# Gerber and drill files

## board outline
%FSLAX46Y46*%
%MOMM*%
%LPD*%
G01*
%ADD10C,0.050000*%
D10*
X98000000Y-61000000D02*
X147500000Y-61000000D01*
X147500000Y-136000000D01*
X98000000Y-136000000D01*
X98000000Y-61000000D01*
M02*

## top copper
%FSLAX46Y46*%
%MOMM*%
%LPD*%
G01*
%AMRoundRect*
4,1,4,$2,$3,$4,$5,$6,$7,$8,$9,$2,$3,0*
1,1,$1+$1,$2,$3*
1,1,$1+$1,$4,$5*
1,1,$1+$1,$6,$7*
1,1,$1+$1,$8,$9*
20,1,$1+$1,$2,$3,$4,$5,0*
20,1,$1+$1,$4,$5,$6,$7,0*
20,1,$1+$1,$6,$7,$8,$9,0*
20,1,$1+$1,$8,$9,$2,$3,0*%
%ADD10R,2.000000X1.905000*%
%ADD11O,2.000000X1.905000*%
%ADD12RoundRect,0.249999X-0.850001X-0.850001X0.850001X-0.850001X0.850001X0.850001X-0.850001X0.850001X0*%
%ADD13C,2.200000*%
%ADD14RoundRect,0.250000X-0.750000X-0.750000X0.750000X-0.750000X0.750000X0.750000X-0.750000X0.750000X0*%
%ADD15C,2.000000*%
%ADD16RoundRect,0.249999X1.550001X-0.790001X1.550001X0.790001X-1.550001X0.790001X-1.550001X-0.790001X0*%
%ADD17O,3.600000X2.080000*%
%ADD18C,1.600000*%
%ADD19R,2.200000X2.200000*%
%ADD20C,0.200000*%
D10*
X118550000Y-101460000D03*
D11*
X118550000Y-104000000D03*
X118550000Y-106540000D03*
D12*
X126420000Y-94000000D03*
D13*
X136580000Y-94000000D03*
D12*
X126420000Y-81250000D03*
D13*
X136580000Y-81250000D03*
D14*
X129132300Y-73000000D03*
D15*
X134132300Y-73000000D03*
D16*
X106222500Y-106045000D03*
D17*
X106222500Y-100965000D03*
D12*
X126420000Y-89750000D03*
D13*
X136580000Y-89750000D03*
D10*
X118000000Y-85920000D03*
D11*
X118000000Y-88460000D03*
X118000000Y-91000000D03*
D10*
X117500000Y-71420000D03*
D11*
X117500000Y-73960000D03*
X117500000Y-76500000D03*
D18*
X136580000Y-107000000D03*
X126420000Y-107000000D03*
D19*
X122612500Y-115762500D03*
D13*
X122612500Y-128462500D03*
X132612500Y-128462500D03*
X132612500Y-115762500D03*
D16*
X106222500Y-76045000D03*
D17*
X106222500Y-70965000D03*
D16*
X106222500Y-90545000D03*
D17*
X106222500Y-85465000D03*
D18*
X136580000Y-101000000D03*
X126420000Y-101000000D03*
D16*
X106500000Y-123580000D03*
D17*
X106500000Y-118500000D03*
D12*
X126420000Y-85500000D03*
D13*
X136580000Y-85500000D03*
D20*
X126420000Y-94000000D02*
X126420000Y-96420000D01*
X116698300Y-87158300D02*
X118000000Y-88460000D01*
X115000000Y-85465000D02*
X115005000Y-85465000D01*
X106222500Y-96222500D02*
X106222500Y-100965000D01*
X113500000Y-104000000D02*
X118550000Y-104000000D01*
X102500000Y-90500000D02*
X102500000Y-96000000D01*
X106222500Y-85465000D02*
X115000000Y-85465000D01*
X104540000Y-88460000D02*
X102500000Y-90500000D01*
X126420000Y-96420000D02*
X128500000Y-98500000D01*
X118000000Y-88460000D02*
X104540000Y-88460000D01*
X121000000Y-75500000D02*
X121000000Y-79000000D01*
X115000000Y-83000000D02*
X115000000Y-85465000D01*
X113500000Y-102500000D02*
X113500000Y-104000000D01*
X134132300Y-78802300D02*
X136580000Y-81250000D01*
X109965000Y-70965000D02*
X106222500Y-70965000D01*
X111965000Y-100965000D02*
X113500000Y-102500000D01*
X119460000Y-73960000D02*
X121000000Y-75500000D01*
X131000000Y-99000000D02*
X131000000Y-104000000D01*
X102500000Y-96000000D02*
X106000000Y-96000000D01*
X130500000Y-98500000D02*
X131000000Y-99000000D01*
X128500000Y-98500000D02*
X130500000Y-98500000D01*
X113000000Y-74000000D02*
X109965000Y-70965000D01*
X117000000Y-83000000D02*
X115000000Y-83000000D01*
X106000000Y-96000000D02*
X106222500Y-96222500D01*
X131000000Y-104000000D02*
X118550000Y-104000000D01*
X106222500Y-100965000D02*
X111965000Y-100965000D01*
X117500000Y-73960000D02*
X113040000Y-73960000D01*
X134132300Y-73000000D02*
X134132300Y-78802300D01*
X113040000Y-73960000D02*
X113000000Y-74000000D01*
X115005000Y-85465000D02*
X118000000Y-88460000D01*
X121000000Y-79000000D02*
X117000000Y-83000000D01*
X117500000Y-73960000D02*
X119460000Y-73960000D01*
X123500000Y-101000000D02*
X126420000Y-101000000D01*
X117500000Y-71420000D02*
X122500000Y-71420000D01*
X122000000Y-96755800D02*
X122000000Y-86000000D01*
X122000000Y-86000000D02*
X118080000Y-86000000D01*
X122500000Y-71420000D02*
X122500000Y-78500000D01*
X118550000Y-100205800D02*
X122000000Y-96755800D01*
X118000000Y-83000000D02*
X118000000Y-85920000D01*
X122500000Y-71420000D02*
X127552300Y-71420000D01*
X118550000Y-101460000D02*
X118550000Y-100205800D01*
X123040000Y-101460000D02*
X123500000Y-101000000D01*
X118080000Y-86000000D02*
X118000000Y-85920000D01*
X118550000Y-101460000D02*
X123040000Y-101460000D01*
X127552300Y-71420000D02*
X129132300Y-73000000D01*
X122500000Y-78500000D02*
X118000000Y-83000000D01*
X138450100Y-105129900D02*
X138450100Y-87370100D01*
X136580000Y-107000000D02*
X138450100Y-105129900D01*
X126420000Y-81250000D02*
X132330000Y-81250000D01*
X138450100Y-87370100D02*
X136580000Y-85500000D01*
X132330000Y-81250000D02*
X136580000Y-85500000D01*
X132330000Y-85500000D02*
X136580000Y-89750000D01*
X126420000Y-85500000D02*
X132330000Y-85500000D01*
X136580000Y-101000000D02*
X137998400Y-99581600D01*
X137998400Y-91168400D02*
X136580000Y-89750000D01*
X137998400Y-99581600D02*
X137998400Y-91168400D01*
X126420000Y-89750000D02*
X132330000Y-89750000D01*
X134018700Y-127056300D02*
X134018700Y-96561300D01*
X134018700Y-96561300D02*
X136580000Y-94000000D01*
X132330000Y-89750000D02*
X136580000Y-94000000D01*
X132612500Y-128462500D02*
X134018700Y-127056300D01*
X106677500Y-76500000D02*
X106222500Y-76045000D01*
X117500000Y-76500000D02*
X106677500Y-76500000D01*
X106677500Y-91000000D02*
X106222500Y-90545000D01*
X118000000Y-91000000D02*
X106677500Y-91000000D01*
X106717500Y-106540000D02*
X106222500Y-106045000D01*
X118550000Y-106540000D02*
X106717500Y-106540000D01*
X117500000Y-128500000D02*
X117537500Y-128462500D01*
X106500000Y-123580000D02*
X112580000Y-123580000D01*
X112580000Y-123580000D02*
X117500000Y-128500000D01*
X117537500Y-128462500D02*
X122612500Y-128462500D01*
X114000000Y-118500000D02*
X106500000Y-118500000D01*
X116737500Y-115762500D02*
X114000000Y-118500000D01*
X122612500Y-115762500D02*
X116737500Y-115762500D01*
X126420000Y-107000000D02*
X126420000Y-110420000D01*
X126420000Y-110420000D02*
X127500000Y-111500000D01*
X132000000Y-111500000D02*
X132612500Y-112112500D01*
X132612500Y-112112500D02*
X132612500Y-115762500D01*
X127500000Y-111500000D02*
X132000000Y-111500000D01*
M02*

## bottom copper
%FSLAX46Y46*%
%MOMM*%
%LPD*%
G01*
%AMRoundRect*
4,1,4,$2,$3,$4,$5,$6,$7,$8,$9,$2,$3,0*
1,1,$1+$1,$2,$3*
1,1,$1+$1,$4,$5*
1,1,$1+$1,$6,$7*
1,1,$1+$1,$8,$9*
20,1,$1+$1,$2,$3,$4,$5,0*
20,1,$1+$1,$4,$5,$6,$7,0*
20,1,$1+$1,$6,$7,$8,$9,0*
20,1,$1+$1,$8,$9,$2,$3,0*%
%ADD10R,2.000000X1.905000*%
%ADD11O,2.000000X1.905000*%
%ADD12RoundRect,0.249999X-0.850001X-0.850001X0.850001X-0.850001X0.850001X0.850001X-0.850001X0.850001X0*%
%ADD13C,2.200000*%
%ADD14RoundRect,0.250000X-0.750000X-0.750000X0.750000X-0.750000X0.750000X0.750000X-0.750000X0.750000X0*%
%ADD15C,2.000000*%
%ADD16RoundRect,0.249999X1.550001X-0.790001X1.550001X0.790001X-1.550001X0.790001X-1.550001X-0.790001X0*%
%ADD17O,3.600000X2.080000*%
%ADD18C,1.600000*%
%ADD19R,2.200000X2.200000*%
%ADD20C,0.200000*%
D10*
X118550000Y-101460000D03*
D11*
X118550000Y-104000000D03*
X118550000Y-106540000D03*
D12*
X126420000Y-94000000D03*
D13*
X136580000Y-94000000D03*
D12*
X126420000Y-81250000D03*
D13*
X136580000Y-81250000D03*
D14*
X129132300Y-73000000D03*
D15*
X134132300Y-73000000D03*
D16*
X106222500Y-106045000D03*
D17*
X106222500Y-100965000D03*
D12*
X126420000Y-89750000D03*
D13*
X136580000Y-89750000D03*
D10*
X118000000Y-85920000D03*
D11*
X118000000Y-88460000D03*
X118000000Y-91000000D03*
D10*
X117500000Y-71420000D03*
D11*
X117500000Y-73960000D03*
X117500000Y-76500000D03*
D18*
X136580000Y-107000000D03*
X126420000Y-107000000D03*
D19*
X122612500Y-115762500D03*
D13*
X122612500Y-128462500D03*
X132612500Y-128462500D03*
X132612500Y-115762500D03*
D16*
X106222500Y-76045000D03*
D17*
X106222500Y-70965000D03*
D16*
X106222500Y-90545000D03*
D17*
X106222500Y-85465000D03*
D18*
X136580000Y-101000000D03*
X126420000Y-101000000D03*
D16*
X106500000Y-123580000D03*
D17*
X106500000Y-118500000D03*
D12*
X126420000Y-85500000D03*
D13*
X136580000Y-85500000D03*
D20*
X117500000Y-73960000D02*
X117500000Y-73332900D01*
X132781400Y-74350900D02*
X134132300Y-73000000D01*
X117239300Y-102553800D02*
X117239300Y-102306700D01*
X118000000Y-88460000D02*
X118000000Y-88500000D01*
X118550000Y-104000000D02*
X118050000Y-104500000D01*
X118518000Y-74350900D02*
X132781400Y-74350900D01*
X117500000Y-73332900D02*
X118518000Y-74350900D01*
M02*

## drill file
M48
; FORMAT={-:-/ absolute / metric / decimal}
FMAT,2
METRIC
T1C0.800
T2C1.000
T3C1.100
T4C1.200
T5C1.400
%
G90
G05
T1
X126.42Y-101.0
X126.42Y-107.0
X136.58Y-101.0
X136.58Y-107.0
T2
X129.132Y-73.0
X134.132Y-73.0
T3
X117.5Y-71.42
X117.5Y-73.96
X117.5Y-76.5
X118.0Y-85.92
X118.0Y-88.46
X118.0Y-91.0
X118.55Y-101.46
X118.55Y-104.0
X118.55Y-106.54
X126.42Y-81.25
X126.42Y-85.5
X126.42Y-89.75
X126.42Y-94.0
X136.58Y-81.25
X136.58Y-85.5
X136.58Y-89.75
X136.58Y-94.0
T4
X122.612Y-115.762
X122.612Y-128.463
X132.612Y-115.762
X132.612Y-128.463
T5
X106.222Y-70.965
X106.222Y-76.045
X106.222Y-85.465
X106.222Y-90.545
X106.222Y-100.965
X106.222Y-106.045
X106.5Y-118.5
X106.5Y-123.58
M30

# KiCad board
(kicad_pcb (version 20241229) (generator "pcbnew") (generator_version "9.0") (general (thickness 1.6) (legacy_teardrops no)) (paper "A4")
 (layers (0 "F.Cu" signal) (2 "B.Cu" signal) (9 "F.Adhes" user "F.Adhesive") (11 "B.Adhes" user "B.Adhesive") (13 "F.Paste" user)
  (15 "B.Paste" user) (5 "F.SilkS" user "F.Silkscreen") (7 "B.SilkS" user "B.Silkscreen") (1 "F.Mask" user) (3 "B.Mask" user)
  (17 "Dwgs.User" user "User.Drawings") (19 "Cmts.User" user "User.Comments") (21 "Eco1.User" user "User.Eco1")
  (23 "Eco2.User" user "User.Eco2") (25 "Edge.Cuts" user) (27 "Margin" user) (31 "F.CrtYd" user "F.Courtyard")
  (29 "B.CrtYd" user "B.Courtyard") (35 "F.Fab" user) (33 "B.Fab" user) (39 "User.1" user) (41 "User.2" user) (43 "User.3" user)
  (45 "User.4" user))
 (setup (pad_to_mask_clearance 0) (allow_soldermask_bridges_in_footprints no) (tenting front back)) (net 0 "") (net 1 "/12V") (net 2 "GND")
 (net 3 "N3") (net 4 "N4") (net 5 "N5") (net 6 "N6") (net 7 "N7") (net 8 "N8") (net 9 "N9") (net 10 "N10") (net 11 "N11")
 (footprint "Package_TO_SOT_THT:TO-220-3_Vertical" (layer "F.Cu") (at 118.55 101.46 -90)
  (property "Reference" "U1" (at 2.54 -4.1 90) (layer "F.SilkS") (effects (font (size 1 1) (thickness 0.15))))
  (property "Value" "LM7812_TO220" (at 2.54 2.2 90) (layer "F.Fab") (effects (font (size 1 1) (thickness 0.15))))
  (pad "1" thru_hole rect (at 0 0 270) (size 1.905 2) (drill 1.1) (layers "*.Cu" "*.Mask") (remove_unused_layers no) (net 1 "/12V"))
  (pad "2" thru_hole oval (at 2.54 0 270) (size 1.905 2) (drill 1.1) (layers "*.Cu" "*.Mask") (remove_unused_layers no) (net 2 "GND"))
  (pad "3" thru_hole oval (at 5.08 0 270) (size 1.905 2) (drill 1.1) (layers "*.Cu" "*.Mask") (remove_unused_layers no) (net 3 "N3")))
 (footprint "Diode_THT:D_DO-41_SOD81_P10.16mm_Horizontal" (layer "F.Cu") (at 126.42 94)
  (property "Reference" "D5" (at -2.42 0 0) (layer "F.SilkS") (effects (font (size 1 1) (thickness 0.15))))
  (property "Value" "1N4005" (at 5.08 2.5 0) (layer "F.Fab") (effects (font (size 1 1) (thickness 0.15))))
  (pad "1" thru_hole roundrect (at 0 0) (size 2.2 2.2) (drill 1.1) (layers "*.Cu" "*.Mask") (remove_unused_layers no)
   (roundrect_rratio 0.113636) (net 2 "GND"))
  (pad "2" thru_hole circle (at 10.16 0) (size 2.2 2.2) (drill 1.1) (layers "*.Cu" "*.Mask") (remove_unused_layers no) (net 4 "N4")))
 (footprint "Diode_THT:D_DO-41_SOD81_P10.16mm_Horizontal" (layer "F.Cu") (at 126.42 81.25)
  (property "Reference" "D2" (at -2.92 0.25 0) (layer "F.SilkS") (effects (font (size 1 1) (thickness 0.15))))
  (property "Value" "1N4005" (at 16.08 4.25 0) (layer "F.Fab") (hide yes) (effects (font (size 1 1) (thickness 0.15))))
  (pad "1" thru_hole roundrect (at 0 0) (size 2.2 2.2) (drill 1.1) (layers "*.Cu" "*.Mask") (remove_unused_layers no)
   (roundrect_rratio 0.113636) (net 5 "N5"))
  (pad "2" thru_hole circle (at 10.16 0) (size 2.2 2.2) (drill 1.1) (layers "*.Cu" "*.Mask") (remove_unused_layers no) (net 2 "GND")))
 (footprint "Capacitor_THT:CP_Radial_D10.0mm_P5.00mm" (layer "F.Cu") (at 129.1323 73)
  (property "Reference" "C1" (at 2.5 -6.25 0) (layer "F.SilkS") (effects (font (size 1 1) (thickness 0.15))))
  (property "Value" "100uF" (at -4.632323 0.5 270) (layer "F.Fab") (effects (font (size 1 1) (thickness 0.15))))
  (pad "1" thru_hole roundrect (at 0 0) (size 2 2) (drill 1) (layers "*.Cu" "*.Mask") (remove_unused_layers no) (roundrect_rratio 0.125)
   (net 1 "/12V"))
  (pad "2" thru_hole circle (at 5 0) (size 2 2) (drill 1) (layers "*.Cu" "*.Mask") (remove_unused_layers no) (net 2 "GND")))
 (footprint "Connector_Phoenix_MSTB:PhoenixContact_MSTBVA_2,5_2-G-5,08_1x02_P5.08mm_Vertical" (layer "F.Cu") (at 106.2225 106.045 90)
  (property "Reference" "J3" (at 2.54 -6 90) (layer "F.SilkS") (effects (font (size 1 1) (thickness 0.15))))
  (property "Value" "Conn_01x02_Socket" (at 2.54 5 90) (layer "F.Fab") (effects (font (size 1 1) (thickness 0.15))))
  (pad "1" thru_hole roundrect (at 0 0 90) (size 2.08 3.6) (drill 1.4) (layers "*.Cu" "*.Mask") (remove_unused_layers no)
   (roundrect_rratio 0.120192) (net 3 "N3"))
  (pad "2" thru_hole oval (at 5.08 0 90) (size 2.08 3.6) (drill 1.4) (layers "*.Cu" "*.Mask") (remove_unused_layers no) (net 2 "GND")))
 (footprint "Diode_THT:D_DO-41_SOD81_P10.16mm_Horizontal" (layer "F.Cu") (at 126.42 89.75)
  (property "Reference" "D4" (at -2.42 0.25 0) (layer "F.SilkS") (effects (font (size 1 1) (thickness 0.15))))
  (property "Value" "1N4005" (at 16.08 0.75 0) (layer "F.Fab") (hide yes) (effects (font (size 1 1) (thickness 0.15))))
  (pad "1" thru_hole roundrect (at 0 0) (size 2.2 2.2) (drill 1.1) (layers "*.Cu" "*.Mask") (remove_unused_layers no)
   (roundrect_rratio 0.113636) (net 4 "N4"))
  (pad "2" thru_hole circle (at 10.16 0) (size 2.2 2.2) (drill 1.1) (layers "*.Cu" "*.Mask") (remove_unused_layers no) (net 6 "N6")))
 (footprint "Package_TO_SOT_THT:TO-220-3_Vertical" (layer "F.Cu") (at 118 85.92 -90)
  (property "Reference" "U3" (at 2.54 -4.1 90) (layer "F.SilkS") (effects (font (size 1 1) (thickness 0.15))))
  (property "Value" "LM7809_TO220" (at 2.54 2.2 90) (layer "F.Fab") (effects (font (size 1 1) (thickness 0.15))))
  (pad "1" thru_hole rect (at 0 0 270) (size 1.905 2) (drill 1.1) (layers "*.Cu" "*.Mask") (remove_unused_layers no) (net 1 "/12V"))
  (pad "2" thru_hole oval (at 2.54 0 270) (size 1.905 2) (drill 1.1) (layers "*.Cu" "*.Mask") (remove_unused_layers no) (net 2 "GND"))
  (pad "3" thru_hole oval (at 5.08 0 270) (size 1.905 2) (drill 1.1) (layers "*.Cu" "*.Mask") (remove_unused_layers no) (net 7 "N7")))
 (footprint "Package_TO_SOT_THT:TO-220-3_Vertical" (layer "F.Cu") (at 117.5 71.42 -90)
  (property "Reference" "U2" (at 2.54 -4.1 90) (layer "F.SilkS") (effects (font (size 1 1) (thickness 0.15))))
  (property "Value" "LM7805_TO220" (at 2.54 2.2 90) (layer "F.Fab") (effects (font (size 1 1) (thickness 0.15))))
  (pad "1" thru_hole rect (at 0 0 270) (size 1.905 2) (drill 1.1) (layers "*.Cu" "*.Mask") (remove_unused_layers no) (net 1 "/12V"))
  (pad "2" thru_hole oval (at 2.54 0 270) (size 1.905 2) (drill 1.1) (layers "*.Cu" "*.Mask") (remove_unused_layers no) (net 2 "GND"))
  (pad "3" thru_hole oval (at 5.08 0 270) (size 1.905 2) (drill 1.1) (layers "*.Cu" "*.Mask") (remove_unused_layers no) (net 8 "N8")))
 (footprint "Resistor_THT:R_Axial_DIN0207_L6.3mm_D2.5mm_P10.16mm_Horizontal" (layer "F.Cu") (at 136.58 107 180)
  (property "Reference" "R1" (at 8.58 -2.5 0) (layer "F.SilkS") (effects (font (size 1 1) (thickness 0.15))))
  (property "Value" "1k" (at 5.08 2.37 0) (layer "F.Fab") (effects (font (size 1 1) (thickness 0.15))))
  (pad "1" thru_hole circle (at 0 0 180) (size 1.6 1.6) (drill 0.8) (layers "*.Cu" "*.Mask") (remove_unused_layers no) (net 5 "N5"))
  (pad "2" thru_hole circle (at 10.16 0 180) (size 1.6 1.6) (drill 0.8) (layers "*.Cu" "*.Mask") (remove_unused_layers no) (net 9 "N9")))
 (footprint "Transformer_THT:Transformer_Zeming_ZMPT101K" (layer "F.Cu") (at 122.6125 115.7625)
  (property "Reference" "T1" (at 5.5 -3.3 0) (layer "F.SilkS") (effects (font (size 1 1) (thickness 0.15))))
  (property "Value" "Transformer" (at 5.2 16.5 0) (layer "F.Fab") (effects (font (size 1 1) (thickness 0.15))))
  (pad "1" thru_hole rect (at 0 0) (size 2.2 2.2) (drill 1.2) (layers "*.Cu" "*.Mask") (remove_unused_layers no) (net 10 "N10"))
  (pad "2" thru_hole circle (at 0 12.7) (size 2.2 2.2) (drill 1.2) (layers "*.Cu" "*.Mask") (remove_unused_layers no) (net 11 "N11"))
  (pad "3" thru_hole circle (at 10 12.7) (size 2.2 2.2) (drill 1.2) (layers "*.Cu" "*.Mask") (remove_unused_layers no) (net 4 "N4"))
  (pad "4" thru_hole circle (at 10 0) (size 2.2 2.2) (drill 1.2) (layers "*.Cu" "*.Mask") (remove_unused_layers no) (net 9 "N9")))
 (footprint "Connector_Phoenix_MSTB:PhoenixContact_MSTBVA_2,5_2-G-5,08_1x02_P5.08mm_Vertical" (layer "F.Cu") (at 106.2225 76.045 90)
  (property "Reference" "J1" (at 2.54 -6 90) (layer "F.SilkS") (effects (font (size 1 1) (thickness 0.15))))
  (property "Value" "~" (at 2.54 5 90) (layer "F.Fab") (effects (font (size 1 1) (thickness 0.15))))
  (pad "1" thru_hole roundrect (at 0 0 90) (size 2.08 3.6) (drill 1.4) (layers "*.Cu" "*.Mask") (remove_unused_layers no)
   (roundrect_rratio 0.120192) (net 8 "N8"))
  (pad "2" thru_hole oval (at 5.08 0 90) (size 2.08 3.6) (drill 1.4) (layers "*.Cu" "*.Mask") (remove_unused_layers no) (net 2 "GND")))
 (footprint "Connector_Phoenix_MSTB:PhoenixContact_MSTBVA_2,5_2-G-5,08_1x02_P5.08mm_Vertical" (layer "F.Cu") (at 106.2225 90.545 90)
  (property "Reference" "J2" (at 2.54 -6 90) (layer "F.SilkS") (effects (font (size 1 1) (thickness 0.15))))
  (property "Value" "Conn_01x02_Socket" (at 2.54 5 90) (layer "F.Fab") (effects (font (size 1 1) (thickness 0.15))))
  (pad "1" thru_hole roundrect (at 0 0 90) (size 2.08 3.6) (drill 1.4) (layers "*.Cu" "*.Mask") (remove_unused_layers no)
   (roundrect_rratio 0.120192) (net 7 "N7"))
  (pad "2" thru_hole oval (at 5.08 0 90) (size 2.08 3.6) (drill 1.4) (layers "*.Cu" "*.Mask") (remove_unused_layers no) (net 2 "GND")))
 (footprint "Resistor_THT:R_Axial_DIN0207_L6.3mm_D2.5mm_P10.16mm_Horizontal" (layer "F.Cu") (at 136.58 101 180)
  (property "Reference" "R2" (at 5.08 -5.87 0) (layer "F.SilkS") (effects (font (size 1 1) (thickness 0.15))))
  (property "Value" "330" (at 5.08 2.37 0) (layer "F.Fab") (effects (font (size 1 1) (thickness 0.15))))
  (pad "1" thru_hole circle (at 0 0 180) (size 1.6 1.6) (drill 0.8) (layers "*.Cu" "*.Mask") (remove_unused_layers no) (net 6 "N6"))
  (pad "2" thru_hole circle (at 10.16 0 180) (size 1.6 1.6) (drill 0.8) (layers "*.Cu" "*.Mask") (remove_unused_layers no) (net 1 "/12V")))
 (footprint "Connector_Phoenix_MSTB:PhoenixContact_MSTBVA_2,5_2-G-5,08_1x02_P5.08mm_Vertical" (layer "F.Cu") (at 106.5 123.58 90)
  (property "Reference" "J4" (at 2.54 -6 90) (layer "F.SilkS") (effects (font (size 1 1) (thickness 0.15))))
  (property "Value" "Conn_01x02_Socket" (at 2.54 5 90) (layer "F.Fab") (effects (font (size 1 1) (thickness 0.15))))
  (pad "1" thru_hole roundrect (at 0 0 90) (size 2.08 3.6) (drill 1.4) (layers "*.Cu" "*.Mask") (remove_unused_layers no)
   (roundrect_rratio 0.120192) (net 11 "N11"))
  (pad "2" thru_hole oval (at 5.08 0 90) (size 2.08 3.6) (drill 1.4) (layers "*.Cu" "*.Mask") (remove_unused_layers no) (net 10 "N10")))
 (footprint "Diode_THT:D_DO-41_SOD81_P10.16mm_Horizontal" (layer "F.Cu") (at 126.42 85.5)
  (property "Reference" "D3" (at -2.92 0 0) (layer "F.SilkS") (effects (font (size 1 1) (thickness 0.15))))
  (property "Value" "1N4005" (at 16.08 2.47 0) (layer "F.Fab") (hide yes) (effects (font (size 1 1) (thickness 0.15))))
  (pad "1" thru_hole roundrect (at 0 0) (size 2.2 2.2) (drill 1.1) (layers "*.Cu" "*.Mask") (remove_unused_layers no)
   (roundrect_rratio 0.113636) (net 6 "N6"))
  (pad "2" thru_hole circle (at 10.16 0) (size 2.2 2.2) (drill 1.1) (layers "*.Cu" "*.Mask") (remove_unused_layers no) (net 5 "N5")))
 (gr_rect (start 98 61) (end 147.5 136) (stroke (width 0.05) (type default)) (fill no) (layer "Edge.Cuts"))
 (segment (start 126.42 94) (end 126.42 96.42) (width 0.2) (layer "F.Cu") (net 2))
 (segment (start 116.6983 87.1583) (end 118 88.46) (width 0.2) (layer "F.Cu") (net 2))
 (segment (start 115 85.465) (end 115.005 85.465) (width 0.2) (layer "F.Cu") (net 2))
 (segment (start 106.2225 96.2225) (end 106.2225 100.965) (width 0.2) (layer "F.Cu") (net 2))
 (segment (start 113.5 104) (end 118.55 104) (width 0.2) (layer "F.Cu") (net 2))
 (segment (start 102.5 90.5) (end 102.5 96) (width 0.2) (layer "F.Cu") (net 2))
 (segment (start 106.2225 85.465) (end 115 85.465) (width 0.2) (layer "F.Cu") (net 2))
 (segment (start 104.54 88.46) (end 102.5 90.5) (width 0.2) (layer "F.Cu") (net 2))
 (segment (start 126.42 96.42) (end 128.5 98.5) (width 0.2) (layer "F.Cu") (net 2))
 (segment (start 118 88.46) (end 104.54 88.46) (width 0.2) (layer "F.Cu") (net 2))
 (segment (start 121 75.5) (end 121 79) (width 0.2) (layer "F.Cu") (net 2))
 (segment (start 115 83) (end 115 85.465) (width 0.2) (layer "F.Cu") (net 2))
 (segment (start 113.5 102.5) (end 113.5 104) (width 0.2) (layer "F.Cu") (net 2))
 (segment (start 134.1323 78.8023) (end 136.58 81.25) (width 0.2) (layer "F.Cu") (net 2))
 (segment (start 109.965 70.965) (end 106.2225 70.965) (width 0.2) (layer "F.Cu") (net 2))
 (segment (start 111.965 100.965) (end 113.5 102.5) (width 0.2) (layer "F.Cu") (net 2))
 (segment (start 119.46 73.96) (end 121 75.5) (width 0.2) (layer "F.Cu") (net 2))
 (segment (start 131 99) (end 131 104) (width 0.2) (layer "F.Cu") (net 2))
 (segment (start 102.5 96) (end 106 96) (width 0.2) (layer "F.Cu") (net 2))
 (segment (start 130.5 98.5) (end 131 99) (width 0.2) (layer "F.Cu") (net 2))
 (segment (start 128.5 98.5) (end 130.5 98.5) (width 0.2) (layer "F.Cu") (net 2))
 (segment (start 113 74) (end 109.965 70.965) (width 0.2) (layer "F.Cu") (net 2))
 (segment (start 117 83) (end 115 83) (width 0.2) (layer "F.Cu") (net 2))
 (segment (start 106 96) (end 106.2225 96.2225) (width 0.2) (layer "F.Cu") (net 2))
 (segment (start 131 104) (end 118.55 104) (width 0.2) (layer "F.Cu") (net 2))
 (segment (start 106.2225 100.965) (end 111.965 100.965) (width 0.2) (layer "F.Cu") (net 2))
 (segment (start 117.5 73.96) (end 113.04 73.96) (width 0.2) (layer "F.Cu") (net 2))
 (segment (start 134.1323 73) (end 134.1323 78.8023) (width 0.2) (layer "F.Cu") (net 2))
 (segment (start 113.04 73.96) (end 113 74) (width 0.2) (layer "F.Cu") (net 2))
 (segment (start 115.005 85.465) (end 118 88.46) (width 0.2) (layer "F.Cu") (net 2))
 (segment (start 121 79) (end 117 83) (width 0.2) (layer "F.Cu") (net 2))
 (segment (start 117.5 73.96) (end 119.46 73.96) (width 0.2) (layer "F.Cu") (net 2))
 (segment (start 117.5 73.96) (end 117.5 73.3329) (width 0.2) (layer "B.Cu") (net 2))
 (segment (start 132.7814 74.3509) (end 134.1323 73) (width 0.2) (layer "B.Cu") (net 2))
 (segment (start 117.2393 102.5538) (end 117.2393 102.3067) (width 0.2) (layer "B.Cu") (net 2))
 (segment (start 118 88.46) (end 118 88.5) (width 0.2) (layer "B.Cu") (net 2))
 (segment (start 118.55 104) (end 118.05 104.5) (width 0.2) (layer "B.Cu") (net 2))
 (segment (start 118.518 74.3509) (end 132.7814 74.3509) (width 0.2) (layer "B.Cu") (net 2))
 (segment (start 117.5 73.3329) (end 118.518 74.3509) (width 0.2) (layer "B.Cu") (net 2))
 (segment (start 123.5 101) (end 126.42 101) (width 0.2) (layer "F.Cu") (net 1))
 (segment (start 117.5 71.42) (end 122.5 71.42) (width 0.2) (layer "F.Cu") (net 1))
 (segment (start 122 96.7558) (end 122 86) (width 0.2) (layer "F.Cu") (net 1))
 (segment (start 122 86) (end 118.08 86) (width 0.2) (layer "F.Cu") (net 1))
 (segment (start 122.5 71.42) (end 122.5 78.5) (width 0.2) (layer "F.Cu") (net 1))
 (segment (start 118.55 100.2058) (end 122 96.7558) (width 0.2) (layer "F.Cu") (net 1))
 (segment (start 118 83) (end 118 85.92) (width 0.2) (layer "F.Cu") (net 1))
 (segment (start 122.5 71.42) (end 127.5523 71.42) (width 0.2) (layer "F.Cu") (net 1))
 (segment (start 118.55 101.46) (end 118.55 100.2058) (width 0.2) (layer "F.Cu") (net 1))
 (segment (start 123.04 101.46) (end 123.5 101) (width 0.2) (layer "F.Cu") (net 1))
 (segment (start 118.08 86) (end 118 85.92) (width 0.2) (layer "F.Cu") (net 1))
 (segment (start 118.55 101.46) (end 123.04 101.46) (width 0.2) (layer "F.Cu") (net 1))
 (segment (start 127.5523 71.42) (end 129.1323 73) (width 0.2) (layer "F.Cu") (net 1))
 (segment (start 122.5 78.5) (end 118 83) (width 0.2) (layer "F.Cu") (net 1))
 (segment (start 138.4501 105.1299) (end 138.4501 87.3701) (width 0.2) (layer "F.Cu") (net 5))
 (segment (start 136.58 107) (end 138.4501 105.1299) (width 0.2) (layer "F.Cu") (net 5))
 (segment (start 126.42 81.25) (end 132.33 81.25) (width 0.2) (layer "F.Cu") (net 5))
 (segment (start 138.4501 87.3701) (end 136.58 85.5) (width 0.2) (layer "F.Cu") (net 5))
 (segment (start 132.33 81.25) (end 136.58 85.5) (width 0.2) (layer "F.Cu") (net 5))
 (segment (start 132.33 85.5) (end 136.58 89.75) (width 0.2) (layer "F.Cu") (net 6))
 (segment (start 126.42 85.5) (end 132.33 85.5) (width 0.2) (layer "F.Cu") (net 6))
 (segment (start 136.58 101) (end 137.9984 99.5816) (width 0.2) (layer "F.Cu") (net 6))
 (segment (start 137.9984 91.1684) (end 136.58 89.75) (width 0.2) (layer "F.Cu") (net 6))
 (segment (start 137.9984 99.5816) (end 137.9984 91.1684) (width 0.2) (layer "F.Cu") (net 6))
 (segment (start 126.42 89.75) (end 132.33 89.75) (width 0.2) (layer "F.Cu") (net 4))
 (segment (start 134.0187 127.0563) (end 134.0187 96.5613) (width 0.2) (layer "F.Cu") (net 4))
 (segment (start 134.0187 96.5613) (end 136.58 94) (width 0.2) (layer "F.Cu") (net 4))
 (segment (start 132.33 89.75) (end 136.58 94) (width 0.2) (layer "F.Cu") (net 4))
 (segment (start 132.6125 128.4625) (end 134.0187 127.0563) (width 0.2) (layer "F.Cu") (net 4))
 (segment (start 106.6775 76.5) (end 106.2225 76.045) (width 0.2) (layer "F.Cu") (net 8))
 (segment (start 117.5 76.5) (end 106.6775 76.5) (width 0.2) (layer "F.Cu") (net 8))
 (segment (start 106.6775 91) (end 106.2225 90.545) (width 0.2) (layer "F.Cu") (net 7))
 (segment (start 118 91) (end 106.6775 91) (width 0.2) (layer "F.Cu") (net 7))
 (segment (start 106.7175 106.54) (end 106.2225 106.045) (width 0.2) (layer "F.Cu") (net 3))
 (segment (start 118.55 106.54) (end 106.7175 106.54) (width 0.2) (layer "F.Cu") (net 3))
 (segment (start 117.5 128.5) (end 117.5375 128.4625) (width 0.2) (layer "F.Cu") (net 11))
 (segment (start 106.5 123.58) (end 112.58 123.58) (width 0.2) (layer "F.Cu") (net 11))
 (segment (start 112.58 123.58) (end 117.5 128.5) (width 0.2) (layer "F.Cu") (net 11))
 (segment (start 117.5375 128.4625) (end 122.6125 128.4625) (width 0.2) (layer "F.Cu") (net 11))
 (segment (start 114 118.5) (end 106.5 118.5) (width 0.2) (layer "F.Cu") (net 10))
 (segment (start 116.7375 115.7625) (end 114 118.5) (width 0.2) (layer "F.Cu") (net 10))
 (segment (start 122.6125 115.7625) (end 116.7375 115.7625) (width 0.2) (layer "F.Cu") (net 10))
 (segment (start 126.42 107) (end 126.42 110.42) (width 0.2) (layer "F.Cu") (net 9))
 (segment (start 126.42 110.42) (end 127.5 111.5) (width 0.2) (layer "F.Cu") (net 9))
 (segment (start 132 111.5) (end 132.6125 112.1125) (width 0.2) (layer "F.Cu") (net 9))
 (segment (start 132.6125 112.1125) (end 132.6125 115.7625) (width 0.2) (layer "F.Cu") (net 9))
 (segment (start 127.5 111.5) (end 132 111.5) (width 0.2) (layer "F.Cu") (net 9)))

